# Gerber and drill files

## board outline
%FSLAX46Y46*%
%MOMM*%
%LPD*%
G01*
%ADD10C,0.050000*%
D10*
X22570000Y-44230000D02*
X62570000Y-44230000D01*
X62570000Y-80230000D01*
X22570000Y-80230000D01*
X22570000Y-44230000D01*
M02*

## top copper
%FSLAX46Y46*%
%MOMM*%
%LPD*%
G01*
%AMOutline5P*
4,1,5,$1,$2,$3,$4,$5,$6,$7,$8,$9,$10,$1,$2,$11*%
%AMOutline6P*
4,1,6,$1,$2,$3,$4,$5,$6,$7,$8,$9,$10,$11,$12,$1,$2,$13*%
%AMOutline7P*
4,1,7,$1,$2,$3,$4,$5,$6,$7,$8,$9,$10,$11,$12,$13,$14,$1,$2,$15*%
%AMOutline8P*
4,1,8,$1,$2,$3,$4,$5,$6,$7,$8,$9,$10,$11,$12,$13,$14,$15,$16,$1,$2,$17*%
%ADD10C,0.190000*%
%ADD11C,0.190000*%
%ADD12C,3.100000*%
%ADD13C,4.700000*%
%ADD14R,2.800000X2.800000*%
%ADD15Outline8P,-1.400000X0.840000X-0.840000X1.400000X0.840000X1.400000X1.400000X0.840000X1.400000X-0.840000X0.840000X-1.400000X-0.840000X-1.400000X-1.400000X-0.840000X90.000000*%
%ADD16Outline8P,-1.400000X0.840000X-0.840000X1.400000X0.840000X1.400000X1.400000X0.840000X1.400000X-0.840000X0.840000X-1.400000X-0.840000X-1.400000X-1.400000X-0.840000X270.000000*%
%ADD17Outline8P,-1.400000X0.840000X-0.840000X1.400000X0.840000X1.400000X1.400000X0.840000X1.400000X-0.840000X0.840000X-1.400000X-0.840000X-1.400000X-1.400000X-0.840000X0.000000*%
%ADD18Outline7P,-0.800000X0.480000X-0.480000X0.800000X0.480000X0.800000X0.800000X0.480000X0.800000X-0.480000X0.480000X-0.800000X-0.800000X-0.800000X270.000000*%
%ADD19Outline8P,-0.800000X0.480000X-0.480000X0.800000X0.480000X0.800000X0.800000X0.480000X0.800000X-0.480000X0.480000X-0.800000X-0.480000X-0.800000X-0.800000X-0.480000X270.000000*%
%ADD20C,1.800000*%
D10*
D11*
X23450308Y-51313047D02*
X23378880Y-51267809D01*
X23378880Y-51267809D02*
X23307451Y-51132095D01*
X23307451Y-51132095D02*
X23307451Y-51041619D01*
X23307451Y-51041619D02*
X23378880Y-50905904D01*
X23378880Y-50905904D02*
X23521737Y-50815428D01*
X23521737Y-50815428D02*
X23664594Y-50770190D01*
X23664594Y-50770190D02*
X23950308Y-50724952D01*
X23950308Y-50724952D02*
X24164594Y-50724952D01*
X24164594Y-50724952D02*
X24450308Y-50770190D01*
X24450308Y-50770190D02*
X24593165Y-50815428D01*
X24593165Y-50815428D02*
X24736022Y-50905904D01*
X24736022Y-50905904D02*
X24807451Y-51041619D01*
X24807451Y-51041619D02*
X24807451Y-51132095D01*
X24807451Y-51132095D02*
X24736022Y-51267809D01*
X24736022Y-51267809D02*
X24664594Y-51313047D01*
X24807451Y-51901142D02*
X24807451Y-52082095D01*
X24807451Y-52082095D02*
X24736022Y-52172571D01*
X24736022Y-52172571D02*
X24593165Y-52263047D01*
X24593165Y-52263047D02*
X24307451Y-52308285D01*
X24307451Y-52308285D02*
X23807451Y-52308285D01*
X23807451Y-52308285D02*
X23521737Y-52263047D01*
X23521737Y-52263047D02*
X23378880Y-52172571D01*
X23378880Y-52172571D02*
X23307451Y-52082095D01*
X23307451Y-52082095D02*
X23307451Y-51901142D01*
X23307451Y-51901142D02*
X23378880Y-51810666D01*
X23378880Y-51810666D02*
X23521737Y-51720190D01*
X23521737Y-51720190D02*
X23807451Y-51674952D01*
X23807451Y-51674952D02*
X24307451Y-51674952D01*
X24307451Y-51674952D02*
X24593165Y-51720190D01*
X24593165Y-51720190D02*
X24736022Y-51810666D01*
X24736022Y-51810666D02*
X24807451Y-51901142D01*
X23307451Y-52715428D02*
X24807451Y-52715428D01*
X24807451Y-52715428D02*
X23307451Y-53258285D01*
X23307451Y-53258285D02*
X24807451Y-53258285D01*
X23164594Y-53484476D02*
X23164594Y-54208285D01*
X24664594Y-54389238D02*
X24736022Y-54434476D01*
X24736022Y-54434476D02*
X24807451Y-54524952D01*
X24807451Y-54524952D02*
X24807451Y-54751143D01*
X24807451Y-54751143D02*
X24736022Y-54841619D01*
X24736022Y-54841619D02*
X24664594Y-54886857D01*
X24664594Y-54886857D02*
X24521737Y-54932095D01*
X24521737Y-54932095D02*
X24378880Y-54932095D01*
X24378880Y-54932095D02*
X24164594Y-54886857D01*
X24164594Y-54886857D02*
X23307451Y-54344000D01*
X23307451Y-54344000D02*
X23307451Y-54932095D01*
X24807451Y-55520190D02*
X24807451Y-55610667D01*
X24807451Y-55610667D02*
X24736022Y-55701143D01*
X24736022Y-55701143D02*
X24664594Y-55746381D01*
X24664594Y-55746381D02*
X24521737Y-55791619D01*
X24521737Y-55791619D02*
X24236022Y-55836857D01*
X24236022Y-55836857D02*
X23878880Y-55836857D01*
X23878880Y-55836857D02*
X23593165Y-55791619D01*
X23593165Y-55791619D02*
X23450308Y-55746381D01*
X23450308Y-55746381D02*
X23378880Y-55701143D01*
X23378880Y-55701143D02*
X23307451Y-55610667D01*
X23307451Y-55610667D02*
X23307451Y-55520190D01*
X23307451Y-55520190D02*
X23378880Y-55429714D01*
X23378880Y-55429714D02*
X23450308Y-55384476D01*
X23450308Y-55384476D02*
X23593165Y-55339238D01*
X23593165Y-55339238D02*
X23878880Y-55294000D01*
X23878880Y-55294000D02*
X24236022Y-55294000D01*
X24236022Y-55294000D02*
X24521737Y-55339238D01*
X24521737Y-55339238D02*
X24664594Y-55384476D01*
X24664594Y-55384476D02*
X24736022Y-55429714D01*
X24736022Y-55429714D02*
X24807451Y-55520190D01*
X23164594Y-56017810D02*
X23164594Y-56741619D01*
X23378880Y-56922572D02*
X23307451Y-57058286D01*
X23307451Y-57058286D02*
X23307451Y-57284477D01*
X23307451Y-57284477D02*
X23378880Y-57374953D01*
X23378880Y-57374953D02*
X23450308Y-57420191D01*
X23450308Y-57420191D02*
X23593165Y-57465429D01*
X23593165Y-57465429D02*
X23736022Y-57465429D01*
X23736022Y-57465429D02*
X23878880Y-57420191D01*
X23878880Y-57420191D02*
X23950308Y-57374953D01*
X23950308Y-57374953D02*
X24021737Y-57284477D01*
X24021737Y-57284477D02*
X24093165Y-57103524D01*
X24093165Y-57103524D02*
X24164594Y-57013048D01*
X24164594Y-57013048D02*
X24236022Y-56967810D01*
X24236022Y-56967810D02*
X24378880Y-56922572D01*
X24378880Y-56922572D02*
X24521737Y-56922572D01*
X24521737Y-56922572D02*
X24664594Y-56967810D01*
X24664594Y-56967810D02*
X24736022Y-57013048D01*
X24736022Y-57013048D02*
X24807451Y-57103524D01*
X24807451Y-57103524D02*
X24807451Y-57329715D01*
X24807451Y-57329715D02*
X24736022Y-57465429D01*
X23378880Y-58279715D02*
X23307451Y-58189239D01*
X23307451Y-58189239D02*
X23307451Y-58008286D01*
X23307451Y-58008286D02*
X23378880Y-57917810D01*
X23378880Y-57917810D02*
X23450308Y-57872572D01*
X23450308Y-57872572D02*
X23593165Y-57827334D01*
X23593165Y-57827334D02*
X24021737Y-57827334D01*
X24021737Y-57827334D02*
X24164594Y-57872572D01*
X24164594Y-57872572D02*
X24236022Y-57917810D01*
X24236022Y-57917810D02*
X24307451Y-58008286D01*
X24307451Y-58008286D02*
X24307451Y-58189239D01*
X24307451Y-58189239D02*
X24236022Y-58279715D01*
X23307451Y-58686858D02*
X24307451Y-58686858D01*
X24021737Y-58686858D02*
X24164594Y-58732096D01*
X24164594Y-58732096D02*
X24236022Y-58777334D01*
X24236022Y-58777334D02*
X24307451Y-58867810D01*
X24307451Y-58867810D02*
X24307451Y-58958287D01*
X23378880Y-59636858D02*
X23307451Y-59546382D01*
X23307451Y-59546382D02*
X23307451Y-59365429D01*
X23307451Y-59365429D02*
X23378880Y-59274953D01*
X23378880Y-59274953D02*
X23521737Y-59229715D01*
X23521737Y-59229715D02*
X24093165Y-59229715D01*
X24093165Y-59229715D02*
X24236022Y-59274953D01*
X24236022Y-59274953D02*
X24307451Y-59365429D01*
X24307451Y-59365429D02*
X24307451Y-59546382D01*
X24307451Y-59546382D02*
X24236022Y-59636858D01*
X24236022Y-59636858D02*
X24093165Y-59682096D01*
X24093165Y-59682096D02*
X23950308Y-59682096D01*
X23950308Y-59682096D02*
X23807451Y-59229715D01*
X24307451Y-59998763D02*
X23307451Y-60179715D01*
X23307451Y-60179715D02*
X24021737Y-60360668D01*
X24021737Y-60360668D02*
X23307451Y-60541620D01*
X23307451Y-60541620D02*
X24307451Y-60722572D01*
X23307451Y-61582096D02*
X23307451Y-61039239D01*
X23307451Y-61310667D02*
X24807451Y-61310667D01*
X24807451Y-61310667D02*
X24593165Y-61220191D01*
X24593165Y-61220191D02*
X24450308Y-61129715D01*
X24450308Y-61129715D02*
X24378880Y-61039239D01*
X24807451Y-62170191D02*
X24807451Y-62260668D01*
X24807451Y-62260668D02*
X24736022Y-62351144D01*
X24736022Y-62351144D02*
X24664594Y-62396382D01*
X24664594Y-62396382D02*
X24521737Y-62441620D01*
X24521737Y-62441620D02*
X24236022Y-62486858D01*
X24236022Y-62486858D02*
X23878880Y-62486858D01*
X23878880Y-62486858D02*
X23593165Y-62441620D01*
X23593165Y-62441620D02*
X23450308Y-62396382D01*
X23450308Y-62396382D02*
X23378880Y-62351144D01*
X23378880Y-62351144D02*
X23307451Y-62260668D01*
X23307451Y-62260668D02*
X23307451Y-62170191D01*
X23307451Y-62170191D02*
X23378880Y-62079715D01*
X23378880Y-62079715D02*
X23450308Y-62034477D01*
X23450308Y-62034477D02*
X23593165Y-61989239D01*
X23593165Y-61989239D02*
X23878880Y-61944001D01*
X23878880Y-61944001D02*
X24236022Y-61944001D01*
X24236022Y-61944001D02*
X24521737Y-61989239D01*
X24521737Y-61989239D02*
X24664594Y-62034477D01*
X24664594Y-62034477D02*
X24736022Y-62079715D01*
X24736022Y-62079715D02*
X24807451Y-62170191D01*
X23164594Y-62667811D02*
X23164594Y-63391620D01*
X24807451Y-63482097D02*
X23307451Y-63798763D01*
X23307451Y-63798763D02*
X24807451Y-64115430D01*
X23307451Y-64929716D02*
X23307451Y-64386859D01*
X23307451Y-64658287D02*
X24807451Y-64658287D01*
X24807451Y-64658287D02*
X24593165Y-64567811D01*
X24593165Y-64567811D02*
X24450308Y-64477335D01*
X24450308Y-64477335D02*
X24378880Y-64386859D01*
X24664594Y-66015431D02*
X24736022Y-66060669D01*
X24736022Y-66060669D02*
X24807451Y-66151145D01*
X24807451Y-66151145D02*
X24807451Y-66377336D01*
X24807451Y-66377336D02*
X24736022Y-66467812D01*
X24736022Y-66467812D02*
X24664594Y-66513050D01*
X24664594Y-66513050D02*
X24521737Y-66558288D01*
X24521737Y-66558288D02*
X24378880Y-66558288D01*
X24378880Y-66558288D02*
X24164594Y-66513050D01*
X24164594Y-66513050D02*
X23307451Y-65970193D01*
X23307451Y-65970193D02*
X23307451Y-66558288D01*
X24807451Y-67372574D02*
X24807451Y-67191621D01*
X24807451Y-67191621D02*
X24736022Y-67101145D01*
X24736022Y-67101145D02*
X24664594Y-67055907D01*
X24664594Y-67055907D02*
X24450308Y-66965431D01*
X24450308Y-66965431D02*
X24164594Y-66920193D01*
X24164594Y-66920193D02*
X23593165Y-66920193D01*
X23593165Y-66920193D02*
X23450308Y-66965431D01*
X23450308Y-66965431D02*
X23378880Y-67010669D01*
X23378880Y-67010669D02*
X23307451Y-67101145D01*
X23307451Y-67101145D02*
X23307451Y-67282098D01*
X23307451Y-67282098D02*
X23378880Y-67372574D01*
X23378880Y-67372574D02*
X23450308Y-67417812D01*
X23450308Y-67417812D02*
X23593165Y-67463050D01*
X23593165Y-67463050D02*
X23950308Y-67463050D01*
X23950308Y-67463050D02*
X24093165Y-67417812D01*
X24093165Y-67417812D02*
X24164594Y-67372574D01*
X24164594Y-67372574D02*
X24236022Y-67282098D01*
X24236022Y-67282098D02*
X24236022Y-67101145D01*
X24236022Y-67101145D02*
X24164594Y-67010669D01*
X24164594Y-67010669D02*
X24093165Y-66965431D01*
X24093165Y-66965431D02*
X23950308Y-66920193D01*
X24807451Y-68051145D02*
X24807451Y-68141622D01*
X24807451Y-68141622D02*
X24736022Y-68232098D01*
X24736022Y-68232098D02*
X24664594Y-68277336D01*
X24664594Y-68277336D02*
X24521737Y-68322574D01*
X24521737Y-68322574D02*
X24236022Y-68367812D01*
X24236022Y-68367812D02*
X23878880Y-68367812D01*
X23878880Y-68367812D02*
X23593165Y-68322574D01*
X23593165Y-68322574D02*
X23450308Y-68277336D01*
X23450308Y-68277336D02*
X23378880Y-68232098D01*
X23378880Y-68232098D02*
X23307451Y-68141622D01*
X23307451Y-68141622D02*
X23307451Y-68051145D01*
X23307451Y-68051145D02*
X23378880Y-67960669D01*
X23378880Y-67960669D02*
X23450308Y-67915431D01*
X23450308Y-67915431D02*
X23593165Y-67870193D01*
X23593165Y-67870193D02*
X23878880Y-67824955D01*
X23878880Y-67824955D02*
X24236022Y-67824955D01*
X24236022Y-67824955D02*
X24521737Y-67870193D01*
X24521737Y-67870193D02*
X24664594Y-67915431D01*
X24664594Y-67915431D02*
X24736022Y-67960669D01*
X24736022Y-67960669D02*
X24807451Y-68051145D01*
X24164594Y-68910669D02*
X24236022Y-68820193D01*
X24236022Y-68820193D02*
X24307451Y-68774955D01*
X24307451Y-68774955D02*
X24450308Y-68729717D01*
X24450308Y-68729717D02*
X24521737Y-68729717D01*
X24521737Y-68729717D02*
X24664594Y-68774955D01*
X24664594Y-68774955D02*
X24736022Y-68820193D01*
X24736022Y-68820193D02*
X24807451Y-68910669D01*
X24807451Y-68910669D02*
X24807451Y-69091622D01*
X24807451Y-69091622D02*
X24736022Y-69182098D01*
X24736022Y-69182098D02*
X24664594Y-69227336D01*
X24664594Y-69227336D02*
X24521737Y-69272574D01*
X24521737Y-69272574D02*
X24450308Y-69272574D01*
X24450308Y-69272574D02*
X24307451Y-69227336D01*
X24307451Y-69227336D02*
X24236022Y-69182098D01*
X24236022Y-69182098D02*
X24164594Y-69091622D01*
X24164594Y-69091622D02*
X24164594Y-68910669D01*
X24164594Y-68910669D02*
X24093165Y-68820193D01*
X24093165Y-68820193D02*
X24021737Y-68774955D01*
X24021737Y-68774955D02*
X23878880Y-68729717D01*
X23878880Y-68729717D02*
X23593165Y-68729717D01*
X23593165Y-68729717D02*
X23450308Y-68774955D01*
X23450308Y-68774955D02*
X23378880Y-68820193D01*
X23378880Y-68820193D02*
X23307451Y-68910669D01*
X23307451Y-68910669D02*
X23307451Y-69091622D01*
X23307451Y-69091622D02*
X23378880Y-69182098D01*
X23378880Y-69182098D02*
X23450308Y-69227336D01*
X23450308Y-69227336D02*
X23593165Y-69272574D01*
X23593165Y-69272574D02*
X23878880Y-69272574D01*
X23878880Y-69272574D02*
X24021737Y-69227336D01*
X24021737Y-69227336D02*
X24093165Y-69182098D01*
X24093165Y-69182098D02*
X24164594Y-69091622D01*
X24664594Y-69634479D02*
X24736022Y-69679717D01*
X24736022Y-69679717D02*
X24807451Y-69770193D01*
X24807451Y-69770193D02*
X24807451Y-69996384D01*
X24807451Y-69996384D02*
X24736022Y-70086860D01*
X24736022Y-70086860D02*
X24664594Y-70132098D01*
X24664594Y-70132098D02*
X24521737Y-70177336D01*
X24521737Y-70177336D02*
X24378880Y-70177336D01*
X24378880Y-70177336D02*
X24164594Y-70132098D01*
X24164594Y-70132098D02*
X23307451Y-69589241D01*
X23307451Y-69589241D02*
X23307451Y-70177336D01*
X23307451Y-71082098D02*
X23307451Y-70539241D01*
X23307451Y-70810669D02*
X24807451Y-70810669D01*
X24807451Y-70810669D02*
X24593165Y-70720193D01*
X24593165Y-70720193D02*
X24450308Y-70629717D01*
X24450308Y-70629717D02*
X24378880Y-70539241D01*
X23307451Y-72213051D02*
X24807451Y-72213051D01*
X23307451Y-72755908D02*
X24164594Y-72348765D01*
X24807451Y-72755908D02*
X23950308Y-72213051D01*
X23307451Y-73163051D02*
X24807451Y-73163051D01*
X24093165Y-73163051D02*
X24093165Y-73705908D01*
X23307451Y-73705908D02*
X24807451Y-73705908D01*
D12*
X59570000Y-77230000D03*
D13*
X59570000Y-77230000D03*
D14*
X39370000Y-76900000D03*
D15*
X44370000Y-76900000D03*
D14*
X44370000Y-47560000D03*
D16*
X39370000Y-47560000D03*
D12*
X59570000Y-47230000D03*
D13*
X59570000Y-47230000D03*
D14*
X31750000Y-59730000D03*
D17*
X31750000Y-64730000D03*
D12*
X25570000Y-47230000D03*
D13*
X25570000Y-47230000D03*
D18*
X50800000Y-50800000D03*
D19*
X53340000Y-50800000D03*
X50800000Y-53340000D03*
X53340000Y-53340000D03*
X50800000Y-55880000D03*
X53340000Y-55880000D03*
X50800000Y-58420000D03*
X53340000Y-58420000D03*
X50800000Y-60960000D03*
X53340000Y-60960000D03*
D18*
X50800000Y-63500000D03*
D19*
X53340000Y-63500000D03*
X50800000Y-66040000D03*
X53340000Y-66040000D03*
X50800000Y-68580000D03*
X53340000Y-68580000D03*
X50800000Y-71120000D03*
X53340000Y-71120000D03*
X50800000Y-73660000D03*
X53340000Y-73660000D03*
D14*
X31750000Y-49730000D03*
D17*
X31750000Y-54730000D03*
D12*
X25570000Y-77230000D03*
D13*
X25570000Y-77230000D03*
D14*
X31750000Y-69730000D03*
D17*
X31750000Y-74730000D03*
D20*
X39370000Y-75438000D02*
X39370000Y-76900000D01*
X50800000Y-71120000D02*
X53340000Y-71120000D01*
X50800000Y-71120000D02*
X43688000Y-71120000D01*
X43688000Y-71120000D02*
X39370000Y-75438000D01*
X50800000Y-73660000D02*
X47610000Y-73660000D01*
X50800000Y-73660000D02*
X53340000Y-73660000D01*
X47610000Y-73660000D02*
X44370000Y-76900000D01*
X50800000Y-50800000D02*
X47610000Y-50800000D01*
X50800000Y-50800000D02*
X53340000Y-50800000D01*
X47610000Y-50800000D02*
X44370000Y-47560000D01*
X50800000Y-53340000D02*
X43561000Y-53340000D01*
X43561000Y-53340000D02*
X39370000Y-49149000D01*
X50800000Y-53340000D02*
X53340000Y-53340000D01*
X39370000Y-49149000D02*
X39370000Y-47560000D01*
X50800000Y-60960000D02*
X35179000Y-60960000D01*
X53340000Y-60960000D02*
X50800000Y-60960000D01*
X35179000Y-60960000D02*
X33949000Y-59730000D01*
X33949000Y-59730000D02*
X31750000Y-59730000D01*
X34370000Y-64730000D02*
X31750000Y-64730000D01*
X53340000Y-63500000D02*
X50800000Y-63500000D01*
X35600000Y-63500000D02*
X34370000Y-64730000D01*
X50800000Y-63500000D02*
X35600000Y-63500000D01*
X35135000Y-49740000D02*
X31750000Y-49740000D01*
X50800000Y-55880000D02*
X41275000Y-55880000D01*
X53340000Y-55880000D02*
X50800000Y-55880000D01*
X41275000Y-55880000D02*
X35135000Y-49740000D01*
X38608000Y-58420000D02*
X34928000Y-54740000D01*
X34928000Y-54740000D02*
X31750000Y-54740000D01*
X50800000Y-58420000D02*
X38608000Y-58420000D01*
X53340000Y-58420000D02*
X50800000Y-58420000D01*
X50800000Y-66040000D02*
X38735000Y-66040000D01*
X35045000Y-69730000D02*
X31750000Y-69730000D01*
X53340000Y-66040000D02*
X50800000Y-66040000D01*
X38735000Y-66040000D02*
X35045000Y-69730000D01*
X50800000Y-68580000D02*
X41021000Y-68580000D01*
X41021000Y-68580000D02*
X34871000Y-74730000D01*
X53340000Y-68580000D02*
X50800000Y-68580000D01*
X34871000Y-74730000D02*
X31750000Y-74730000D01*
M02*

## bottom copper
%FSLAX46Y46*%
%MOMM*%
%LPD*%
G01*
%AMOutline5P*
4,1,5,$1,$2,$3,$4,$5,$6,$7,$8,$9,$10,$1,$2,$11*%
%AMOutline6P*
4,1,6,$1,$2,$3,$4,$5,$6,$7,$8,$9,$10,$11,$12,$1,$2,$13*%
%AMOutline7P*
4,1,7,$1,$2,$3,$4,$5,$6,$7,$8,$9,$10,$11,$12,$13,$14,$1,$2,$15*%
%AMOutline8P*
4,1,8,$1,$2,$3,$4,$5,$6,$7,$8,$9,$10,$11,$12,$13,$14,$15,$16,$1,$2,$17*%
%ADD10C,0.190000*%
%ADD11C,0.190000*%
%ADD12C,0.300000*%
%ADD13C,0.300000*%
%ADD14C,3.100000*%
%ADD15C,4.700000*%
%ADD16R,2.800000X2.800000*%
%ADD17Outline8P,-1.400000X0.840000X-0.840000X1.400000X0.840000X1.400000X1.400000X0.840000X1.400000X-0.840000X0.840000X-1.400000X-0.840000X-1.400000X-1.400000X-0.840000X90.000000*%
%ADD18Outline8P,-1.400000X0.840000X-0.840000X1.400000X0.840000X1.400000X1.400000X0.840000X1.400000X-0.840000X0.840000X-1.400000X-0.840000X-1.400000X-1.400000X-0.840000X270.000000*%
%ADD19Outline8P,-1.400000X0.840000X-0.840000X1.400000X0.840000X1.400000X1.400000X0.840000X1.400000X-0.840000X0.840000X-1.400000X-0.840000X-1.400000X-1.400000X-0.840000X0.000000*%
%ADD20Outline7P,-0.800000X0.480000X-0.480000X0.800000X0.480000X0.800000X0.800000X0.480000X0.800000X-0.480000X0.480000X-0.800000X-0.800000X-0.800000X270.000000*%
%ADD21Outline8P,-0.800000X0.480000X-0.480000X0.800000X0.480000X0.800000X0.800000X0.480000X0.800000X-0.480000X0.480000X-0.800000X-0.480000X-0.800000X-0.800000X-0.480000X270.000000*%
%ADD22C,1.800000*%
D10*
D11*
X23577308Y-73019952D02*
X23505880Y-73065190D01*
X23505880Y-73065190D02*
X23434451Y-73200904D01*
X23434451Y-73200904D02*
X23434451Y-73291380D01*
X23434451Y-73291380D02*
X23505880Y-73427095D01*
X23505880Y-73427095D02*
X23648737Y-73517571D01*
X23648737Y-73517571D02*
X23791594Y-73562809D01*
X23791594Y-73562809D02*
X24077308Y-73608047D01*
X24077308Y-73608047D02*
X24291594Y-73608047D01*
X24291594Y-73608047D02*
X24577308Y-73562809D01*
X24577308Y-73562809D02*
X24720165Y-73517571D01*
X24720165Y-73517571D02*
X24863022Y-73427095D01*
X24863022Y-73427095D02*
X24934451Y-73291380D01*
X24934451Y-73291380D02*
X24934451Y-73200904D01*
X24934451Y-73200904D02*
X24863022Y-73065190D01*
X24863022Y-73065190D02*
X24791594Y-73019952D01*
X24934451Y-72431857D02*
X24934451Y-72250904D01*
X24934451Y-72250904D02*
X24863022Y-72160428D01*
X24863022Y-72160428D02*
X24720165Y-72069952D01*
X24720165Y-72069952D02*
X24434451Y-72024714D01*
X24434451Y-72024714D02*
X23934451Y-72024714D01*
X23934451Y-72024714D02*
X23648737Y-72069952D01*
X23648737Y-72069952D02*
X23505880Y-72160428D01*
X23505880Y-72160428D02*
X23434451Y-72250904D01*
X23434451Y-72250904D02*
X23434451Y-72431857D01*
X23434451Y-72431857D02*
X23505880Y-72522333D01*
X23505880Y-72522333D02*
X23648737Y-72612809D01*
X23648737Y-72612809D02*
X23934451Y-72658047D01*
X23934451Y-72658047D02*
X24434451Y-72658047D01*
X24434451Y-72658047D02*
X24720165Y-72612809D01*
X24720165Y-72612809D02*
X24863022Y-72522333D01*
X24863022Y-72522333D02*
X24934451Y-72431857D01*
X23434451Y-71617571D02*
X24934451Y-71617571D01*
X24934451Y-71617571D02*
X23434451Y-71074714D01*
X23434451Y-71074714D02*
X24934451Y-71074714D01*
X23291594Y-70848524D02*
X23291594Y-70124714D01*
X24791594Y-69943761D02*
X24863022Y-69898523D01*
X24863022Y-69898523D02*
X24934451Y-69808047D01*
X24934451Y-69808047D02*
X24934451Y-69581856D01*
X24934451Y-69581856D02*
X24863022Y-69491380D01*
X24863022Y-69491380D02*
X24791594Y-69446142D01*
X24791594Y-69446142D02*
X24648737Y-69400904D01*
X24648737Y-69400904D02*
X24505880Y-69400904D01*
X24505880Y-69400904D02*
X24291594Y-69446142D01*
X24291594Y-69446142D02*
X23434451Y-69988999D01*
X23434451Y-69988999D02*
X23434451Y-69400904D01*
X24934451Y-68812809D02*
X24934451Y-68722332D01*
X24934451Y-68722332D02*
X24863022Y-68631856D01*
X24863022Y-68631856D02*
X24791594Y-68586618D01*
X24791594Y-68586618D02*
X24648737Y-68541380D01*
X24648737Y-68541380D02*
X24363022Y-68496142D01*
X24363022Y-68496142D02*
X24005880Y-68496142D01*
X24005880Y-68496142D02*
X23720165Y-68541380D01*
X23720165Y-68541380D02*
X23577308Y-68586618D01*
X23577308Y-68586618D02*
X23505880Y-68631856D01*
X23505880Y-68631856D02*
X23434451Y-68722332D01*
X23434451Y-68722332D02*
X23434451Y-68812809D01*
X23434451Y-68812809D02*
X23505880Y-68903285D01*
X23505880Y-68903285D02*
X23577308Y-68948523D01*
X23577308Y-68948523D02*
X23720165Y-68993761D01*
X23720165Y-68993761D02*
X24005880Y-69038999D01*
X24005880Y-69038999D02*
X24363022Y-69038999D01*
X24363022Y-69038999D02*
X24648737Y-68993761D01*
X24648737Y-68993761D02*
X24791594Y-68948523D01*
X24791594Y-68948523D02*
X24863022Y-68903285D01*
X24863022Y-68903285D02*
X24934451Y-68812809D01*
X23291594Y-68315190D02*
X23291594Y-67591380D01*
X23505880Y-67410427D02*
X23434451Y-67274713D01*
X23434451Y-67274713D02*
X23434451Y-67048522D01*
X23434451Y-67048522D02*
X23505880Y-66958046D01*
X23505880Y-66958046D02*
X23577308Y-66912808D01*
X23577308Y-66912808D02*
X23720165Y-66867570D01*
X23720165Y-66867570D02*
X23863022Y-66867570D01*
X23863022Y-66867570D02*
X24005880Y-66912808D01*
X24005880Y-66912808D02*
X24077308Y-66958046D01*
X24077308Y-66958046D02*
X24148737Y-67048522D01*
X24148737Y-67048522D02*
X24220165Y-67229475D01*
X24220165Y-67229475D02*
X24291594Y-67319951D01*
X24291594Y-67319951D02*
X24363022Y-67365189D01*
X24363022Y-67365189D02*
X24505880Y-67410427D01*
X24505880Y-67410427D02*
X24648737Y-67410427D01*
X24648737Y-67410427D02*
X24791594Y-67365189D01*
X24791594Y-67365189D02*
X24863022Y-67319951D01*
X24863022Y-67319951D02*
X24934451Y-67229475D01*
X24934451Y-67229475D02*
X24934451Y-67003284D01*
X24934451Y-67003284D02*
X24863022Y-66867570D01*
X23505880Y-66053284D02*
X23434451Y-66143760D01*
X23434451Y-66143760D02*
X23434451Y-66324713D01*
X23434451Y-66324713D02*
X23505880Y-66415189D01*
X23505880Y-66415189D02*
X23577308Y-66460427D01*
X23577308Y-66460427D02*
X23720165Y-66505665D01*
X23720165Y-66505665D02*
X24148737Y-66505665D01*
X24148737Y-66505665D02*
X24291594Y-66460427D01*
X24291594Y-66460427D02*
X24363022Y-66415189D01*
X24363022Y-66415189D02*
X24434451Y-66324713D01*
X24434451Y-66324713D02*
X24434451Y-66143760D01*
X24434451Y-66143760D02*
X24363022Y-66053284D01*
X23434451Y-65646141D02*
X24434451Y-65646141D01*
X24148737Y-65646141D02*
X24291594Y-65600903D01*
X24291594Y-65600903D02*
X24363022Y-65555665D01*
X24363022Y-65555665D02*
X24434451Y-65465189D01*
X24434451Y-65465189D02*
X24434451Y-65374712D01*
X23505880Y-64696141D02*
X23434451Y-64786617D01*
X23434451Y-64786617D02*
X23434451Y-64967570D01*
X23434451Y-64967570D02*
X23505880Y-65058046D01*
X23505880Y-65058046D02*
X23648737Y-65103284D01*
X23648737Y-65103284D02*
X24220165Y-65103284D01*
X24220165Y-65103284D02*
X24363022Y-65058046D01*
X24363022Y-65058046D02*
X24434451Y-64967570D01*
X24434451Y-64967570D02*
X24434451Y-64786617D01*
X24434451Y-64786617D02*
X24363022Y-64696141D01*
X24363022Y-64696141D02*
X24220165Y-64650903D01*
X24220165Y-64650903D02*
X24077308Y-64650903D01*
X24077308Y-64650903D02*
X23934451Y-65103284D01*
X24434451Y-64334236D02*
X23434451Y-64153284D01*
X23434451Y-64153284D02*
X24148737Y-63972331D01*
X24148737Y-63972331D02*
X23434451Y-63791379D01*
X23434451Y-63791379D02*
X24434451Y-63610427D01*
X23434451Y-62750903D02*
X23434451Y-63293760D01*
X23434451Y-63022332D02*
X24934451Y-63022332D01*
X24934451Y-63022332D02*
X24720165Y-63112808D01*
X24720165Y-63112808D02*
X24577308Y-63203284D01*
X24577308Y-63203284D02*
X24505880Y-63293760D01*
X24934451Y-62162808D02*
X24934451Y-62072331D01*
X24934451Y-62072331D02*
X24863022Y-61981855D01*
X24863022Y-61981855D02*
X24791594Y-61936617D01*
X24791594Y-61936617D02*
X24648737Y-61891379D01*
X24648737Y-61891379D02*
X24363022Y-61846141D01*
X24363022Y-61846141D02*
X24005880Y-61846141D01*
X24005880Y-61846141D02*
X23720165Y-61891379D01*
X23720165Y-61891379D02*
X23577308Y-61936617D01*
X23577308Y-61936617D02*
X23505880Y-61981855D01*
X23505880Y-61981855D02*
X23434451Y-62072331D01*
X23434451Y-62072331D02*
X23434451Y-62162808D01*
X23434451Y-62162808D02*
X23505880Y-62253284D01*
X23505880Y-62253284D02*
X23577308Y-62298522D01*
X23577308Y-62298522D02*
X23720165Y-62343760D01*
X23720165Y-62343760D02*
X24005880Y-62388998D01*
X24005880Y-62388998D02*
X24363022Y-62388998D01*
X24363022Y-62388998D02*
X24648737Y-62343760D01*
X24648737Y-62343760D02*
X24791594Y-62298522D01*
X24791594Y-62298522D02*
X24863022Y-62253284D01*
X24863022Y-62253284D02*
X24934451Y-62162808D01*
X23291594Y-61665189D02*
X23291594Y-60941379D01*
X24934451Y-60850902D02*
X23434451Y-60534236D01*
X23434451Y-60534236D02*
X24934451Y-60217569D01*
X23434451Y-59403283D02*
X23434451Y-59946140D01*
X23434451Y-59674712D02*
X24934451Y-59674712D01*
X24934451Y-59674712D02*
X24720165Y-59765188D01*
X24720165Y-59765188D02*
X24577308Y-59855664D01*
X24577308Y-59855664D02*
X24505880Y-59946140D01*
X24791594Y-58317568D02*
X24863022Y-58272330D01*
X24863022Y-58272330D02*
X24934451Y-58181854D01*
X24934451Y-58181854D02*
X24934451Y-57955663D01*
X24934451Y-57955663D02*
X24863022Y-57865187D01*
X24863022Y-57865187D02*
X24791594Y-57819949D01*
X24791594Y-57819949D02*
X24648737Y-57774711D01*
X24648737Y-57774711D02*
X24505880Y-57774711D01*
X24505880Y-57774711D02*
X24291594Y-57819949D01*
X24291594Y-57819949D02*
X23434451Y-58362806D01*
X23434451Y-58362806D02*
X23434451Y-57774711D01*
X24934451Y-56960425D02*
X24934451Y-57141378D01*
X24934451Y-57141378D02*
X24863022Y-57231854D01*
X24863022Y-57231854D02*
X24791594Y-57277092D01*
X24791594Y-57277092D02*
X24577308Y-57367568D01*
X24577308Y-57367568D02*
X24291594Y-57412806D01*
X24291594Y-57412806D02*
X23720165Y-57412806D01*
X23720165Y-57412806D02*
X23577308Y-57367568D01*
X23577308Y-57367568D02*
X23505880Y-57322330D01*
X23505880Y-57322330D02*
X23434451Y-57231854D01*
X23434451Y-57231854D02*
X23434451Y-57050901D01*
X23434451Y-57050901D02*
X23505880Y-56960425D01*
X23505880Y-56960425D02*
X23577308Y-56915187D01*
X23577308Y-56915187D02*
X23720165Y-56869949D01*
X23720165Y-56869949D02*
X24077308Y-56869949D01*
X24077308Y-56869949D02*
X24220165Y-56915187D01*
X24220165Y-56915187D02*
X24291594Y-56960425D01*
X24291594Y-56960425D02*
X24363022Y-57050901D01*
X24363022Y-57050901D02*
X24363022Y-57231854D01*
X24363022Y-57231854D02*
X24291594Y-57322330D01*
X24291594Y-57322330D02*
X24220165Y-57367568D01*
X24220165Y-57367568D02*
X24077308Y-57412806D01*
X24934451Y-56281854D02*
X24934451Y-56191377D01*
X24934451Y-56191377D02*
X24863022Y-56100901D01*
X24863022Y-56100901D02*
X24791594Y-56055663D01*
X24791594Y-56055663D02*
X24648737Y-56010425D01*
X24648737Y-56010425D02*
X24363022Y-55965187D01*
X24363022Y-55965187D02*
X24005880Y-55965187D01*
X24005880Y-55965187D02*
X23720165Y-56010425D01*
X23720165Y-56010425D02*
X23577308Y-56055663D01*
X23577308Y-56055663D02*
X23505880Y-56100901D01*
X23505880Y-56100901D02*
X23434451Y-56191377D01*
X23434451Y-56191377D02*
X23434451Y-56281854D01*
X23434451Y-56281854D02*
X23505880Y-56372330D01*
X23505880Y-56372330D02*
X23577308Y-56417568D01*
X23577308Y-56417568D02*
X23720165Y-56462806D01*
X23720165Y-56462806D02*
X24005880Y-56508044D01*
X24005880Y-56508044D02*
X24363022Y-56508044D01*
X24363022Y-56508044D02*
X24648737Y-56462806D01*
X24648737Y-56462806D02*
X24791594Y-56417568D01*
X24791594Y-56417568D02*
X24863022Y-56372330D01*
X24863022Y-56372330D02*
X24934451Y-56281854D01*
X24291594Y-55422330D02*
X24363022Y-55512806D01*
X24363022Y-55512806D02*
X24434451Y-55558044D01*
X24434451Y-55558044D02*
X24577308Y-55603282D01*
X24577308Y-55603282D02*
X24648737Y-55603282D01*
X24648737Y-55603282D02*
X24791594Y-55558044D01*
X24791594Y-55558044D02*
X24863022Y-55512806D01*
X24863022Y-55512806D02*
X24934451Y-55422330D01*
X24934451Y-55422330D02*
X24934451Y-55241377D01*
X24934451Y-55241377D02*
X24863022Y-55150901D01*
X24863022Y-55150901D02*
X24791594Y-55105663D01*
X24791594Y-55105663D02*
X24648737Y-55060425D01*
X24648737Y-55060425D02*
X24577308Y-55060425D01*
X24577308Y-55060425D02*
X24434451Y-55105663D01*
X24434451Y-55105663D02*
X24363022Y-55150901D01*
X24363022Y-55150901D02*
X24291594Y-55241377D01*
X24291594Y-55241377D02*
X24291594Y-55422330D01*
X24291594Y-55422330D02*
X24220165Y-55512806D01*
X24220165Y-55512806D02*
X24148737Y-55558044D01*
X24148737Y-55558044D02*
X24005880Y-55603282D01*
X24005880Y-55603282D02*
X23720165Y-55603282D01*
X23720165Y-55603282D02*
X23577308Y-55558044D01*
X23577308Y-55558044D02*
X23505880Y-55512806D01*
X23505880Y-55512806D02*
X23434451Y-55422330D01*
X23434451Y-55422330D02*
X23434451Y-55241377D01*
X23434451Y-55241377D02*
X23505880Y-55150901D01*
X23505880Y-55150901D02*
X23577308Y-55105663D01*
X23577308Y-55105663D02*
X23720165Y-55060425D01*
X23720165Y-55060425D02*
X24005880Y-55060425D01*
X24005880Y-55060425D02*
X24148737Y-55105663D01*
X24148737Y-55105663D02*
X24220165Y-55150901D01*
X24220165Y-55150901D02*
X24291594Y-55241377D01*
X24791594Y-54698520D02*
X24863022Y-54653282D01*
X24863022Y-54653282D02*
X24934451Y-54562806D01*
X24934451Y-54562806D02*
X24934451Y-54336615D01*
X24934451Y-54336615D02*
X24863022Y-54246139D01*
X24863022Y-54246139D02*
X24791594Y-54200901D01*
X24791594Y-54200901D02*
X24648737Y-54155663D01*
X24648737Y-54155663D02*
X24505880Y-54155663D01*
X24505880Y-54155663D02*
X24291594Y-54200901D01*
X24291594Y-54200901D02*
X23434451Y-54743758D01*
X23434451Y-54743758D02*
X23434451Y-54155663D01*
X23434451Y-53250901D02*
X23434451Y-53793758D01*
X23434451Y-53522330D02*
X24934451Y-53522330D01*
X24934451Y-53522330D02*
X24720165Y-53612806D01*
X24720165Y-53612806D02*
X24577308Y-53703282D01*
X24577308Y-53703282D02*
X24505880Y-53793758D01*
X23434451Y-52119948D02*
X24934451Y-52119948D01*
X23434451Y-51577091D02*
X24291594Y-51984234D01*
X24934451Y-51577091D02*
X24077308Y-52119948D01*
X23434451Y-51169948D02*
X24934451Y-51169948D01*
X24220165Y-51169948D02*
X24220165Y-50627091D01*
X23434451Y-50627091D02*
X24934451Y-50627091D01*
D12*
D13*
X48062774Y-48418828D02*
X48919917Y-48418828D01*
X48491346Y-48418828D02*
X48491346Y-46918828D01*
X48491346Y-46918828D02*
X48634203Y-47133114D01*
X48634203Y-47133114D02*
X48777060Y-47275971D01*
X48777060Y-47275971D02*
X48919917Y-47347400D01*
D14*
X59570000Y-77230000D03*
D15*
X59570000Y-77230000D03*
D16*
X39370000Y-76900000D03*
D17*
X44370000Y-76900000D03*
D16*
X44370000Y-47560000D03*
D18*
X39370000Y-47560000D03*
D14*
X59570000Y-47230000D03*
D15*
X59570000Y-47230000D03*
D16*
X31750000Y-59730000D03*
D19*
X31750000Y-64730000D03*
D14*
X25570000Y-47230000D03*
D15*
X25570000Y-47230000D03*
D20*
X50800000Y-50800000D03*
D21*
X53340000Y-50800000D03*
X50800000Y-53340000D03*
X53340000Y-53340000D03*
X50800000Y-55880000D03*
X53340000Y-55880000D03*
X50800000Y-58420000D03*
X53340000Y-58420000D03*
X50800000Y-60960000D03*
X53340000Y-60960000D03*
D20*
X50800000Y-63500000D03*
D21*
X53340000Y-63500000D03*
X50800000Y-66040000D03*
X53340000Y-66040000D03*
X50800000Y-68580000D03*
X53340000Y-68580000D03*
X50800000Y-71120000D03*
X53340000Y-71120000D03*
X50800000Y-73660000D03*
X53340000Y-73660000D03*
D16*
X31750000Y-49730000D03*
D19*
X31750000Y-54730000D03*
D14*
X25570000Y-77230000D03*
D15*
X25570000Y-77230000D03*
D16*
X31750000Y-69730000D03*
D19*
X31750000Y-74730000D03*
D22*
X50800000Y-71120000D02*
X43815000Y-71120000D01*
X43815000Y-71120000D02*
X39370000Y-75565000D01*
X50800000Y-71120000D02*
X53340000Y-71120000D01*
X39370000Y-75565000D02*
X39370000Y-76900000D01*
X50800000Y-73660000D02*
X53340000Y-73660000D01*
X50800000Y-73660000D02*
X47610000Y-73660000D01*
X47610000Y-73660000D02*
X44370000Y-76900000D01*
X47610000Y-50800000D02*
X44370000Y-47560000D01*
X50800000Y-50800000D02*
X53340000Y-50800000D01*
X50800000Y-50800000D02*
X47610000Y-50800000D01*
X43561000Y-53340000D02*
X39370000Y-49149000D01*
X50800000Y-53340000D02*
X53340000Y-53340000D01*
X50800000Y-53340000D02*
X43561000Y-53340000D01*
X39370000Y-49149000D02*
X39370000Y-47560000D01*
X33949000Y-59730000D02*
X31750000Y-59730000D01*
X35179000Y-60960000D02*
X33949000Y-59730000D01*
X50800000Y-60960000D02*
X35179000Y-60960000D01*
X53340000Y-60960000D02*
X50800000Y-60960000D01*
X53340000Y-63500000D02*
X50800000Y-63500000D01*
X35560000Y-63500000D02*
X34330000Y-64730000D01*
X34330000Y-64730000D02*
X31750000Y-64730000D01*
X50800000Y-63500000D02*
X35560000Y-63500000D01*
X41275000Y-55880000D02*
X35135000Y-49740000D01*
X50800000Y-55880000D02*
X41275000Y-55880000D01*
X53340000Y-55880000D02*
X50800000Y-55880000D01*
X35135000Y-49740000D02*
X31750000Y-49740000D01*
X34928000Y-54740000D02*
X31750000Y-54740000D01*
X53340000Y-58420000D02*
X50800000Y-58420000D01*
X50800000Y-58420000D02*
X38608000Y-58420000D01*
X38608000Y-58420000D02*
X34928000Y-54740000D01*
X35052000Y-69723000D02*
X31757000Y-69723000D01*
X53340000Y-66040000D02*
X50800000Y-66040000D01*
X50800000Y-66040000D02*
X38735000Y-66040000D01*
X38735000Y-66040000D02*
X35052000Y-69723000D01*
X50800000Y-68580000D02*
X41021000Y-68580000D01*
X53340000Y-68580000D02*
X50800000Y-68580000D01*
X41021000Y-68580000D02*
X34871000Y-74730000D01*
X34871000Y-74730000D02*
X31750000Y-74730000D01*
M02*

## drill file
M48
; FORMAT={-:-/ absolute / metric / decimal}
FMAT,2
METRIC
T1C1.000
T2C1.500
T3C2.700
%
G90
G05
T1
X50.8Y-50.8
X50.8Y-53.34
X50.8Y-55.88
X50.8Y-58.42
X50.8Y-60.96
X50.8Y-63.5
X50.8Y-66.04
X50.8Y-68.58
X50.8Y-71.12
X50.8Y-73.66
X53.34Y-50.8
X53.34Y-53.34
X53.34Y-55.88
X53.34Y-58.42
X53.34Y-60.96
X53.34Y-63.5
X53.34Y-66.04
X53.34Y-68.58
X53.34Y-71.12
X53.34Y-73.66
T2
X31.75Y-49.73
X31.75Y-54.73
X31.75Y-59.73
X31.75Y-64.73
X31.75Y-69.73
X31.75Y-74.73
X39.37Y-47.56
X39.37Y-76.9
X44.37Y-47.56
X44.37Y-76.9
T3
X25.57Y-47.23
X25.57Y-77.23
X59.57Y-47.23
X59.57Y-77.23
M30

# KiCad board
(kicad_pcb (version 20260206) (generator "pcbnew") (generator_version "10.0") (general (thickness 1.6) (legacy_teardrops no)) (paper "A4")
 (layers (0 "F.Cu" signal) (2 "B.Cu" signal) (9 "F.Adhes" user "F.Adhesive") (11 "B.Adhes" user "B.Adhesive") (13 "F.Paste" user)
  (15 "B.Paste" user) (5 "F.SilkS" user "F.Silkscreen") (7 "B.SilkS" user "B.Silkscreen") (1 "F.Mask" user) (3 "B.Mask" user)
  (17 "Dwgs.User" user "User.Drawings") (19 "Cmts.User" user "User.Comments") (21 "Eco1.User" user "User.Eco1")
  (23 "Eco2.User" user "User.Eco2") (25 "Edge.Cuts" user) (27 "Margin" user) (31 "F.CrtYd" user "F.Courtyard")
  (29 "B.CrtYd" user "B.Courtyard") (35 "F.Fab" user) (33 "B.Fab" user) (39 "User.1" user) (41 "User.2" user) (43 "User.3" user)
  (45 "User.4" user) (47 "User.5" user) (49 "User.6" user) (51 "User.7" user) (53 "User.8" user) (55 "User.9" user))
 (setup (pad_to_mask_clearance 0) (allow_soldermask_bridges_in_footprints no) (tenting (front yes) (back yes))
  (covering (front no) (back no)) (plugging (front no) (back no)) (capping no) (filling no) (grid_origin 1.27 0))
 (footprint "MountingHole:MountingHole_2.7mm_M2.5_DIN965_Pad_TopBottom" (layer "F.Cu") (at 59.57 77.23)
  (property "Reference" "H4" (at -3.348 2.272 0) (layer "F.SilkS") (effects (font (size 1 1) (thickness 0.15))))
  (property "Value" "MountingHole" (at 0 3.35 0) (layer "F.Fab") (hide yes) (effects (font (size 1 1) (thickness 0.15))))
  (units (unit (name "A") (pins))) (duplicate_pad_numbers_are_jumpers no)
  (pad "1" thru_hole circle (at 0 0) (size 3.1 3.1) (drill 2.7) (layers "*.Cu" "*.Mask") (remove_unused_layers no))
  (pad "1" connect circle (at 0 0) (size 4.7 4.7) (layers "F.Cu" "F.Mask"))
  (pad "1" connect circle (at 0 0) (size 4.7 4.7) (layers "B.Cu" "B.Mask")))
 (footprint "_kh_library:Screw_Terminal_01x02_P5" (layer "F.Cu") (at 39.37 76.9 90)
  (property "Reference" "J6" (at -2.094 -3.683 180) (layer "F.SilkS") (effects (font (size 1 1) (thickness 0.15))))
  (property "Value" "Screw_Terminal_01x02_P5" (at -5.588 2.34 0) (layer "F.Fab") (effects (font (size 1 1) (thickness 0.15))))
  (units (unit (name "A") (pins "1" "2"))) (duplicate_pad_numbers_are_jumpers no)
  (pad "1" thru_hole rect (at 0 0 90) (size 2.8 2.8) (drill 1.5) (layers "*.Cu" "*.Mask") (remove_unused_layers no) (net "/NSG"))
  (pad "2" thru_hole roundrect (at 0 5 90) (size 2.8 2.8) (drill 1.5) (layers "*.Cu" "*.Mask") (remove_unused_layers no)
   (roundrect_rratio 0) (chamfer_ratio 0.2) (chamfer top_left top_right bottom_left bottom_right) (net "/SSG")))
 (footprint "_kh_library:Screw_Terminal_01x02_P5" (layer "F.Cu") (at 44.37 47.56 -90)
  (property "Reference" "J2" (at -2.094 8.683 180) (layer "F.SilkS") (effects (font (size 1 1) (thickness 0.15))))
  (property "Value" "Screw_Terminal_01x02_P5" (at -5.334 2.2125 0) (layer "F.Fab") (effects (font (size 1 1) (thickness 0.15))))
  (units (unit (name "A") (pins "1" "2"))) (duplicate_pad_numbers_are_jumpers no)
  (pad "1" thru_hole rect (at 0 0 270) (size 2.8 2.8) (drill 1.5) (layers "*.Cu" "*.Mask") (remove_unused_layers no) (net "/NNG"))
  (pad "2" thru_hole roundrect (at 0 5 270) (size 2.8 2.8) (drill 1.5) (layers "*.Cu" "*.Mask") (remove_unused_layers no)
   (roundrect_rratio 0) (chamfer_ratio 0.2) (chamfer top_left top_right bottom_left bottom_right) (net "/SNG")))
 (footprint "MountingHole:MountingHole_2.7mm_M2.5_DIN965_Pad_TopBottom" (layer "F.Cu") (at 59.57 47.23)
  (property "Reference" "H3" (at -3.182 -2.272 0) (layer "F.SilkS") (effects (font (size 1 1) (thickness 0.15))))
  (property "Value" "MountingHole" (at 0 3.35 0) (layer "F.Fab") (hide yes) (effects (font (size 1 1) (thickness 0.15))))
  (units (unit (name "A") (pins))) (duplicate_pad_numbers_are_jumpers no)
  (pad "1" thru_hole circle (at 0 0) (size 3.1 3.1) (drill 2.7) (layers "*.Cu" "*.Mask") (remove_unused_layers no))
  (pad "1" connect circle (at 0 0) (size 4.7 4.7) (layers "F.Cu" "F.Mask"))
  (pad "1" connect circle (at 0 0) (size 4.7 4.7) (layers "B.Cu" "B.Mask")))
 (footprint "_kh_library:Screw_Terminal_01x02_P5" (layer "F.Cu") (at 31.75 59.73)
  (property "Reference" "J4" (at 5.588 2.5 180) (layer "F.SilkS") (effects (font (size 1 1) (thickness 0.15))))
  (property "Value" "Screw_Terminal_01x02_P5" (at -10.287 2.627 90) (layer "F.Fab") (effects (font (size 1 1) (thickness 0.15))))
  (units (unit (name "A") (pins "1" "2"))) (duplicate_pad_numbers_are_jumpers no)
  (pad "1" thru_hole rect (at 0 0) (size 2.8 2.8) (drill 1.5) (layers "*.Cu" "*.Mask") (remove_unused_layers no) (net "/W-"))
  (pad "2" thru_hole roundrect (at 0 5) (size 2.8 2.8) (drill 1.5) (layers "*.Cu" "*.Mask") (remove_unused_layers no) (roundrect_rratio 0)
   (chamfer_ratio 0.2) (chamfer top_left top_right bottom_left bottom_right) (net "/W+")))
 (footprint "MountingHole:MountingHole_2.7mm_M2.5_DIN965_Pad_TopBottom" (layer "F.Cu") (at 25.57 47.23)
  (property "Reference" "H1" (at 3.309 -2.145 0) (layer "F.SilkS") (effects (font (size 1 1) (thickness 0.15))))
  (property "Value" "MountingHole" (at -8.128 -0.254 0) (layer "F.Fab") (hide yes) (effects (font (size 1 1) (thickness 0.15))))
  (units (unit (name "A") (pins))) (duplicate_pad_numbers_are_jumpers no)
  (pad "1" thru_hole circle (at 0 0) (size 3.1 3.1) (drill 2.7) (layers "*.Cu" "*.Mask") (remove_unused_layers no))
  (pad "1" connect circle (at 0 0) (size 4.7 4.7) (layers "F.Cu" "F.Mask"))
  (pad "1" connect circle (at 0 0) (size 4.7 4.7) (layers "B.Cu" "B.Mask")))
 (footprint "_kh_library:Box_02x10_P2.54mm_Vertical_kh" (layer "F.Cu") (at 50.8 50.8 -90)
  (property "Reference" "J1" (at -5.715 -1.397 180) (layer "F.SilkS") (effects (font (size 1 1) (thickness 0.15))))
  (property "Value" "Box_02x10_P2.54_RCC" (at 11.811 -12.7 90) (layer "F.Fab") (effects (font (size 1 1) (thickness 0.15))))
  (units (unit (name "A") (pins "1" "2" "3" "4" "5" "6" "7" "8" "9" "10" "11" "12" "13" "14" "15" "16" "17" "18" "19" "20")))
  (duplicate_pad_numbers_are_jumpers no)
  (pad "1" thru_hole roundrect (at 0 0 270) (size 1.6 1.6) (drill 1) (layers "*.Cu" "*.Mask") (remove_unused_layers no) (roundrect_rratio 0)
   (chamfer_ratio 0.2) (chamfer top_left top_right bottom_right) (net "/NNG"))
  (pad "2" thru_hole roundrect (at 0 -2.54 270) (size 1.6 1.6) (drill 1) (layers "*.Cu" "*.Mask") (remove_unused_layers no)
   (roundrect_rratio 0) (chamfer_ratio 0.2) (chamfer top_left top_right bottom_left bottom_right) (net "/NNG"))
  (pad "3" thru_hole roundrect (at 2.54 0 270) (size 1.6 1.6) (drill 1) (layers "*.Cu" "*.Mask") (remove_unused_layers no)
   (roundrect_rratio 0) (chamfer_ratio 0.2) (chamfer top_left top_right bottom_left bottom_right) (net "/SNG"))
  (pad "4" thru_hole roundrect (at 2.54 -2.54 270) (size 1.6 1.6) (drill 1) (layers "*.Cu" "*.Mask") (remove_unused_layers no)
   (roundrect_rratio 0) (chamfer_ratio 0.2) (chamfer top_left top_right bottom_left bottom_right) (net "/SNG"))
  (pad "5" thru_hole roundrect (at 5.08 0 270) (size 1.6 1.6) (drill 1) (layers "*.Cu" "*.Mask") (remove_unused_layers no)
   (roundrect_rratio 0) (chamfer_ratio 0.2) (chamfer top_left top_right bottom_left bottom_right) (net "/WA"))
  (pad "6" thru_hole roundrect (at 5.08 -2.54 270) (size 1.6 1.6) (drill 1) (layers "*.Cu" "*.Mask") (remove_unused_layers no)
   (roundrect_rratio 0) (chamfer_ratio 0.2) (chamfer top_left top_right bottom_left bottom_right) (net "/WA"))
  (pad "7" thru_hole roundrect (at 7.62 0 270) (size 1.6 1.6) (drill 1) (layers "*.Cu" "*.Mask") (remove_unused_layers no)
   (roundrect_rratio 0) (chamfer_ratio 0.2) (chamfer top_left top_right bottom_left bottom_right) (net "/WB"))
  (pad "8" thru_hole roundrect (at 7.62 -2.54 270) (size 1.6 1.6) (drill 1) (layers "*.Cu" "*.Mask") (remove_unused_layers no)
   (roundrect_rratio 0) (chamfer_ratio 0.2) (chamfer top_left top_right bottom_left bottom_right) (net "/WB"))
  (pad "9" thru_hole roundrect (at 10.16 0 270) (size 1.6 1.6) (drill 1) (layers "*.Cu" "*.Mask") (remove_unused_layers no)
   (roundrect_rratio 0) (chamfer_ratio 0.2) (chamfer top_left top_right bottom_left bottom_right) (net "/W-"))
  (pad "10" thru_hole roundrect (at 10.16 -2.54 270) (size 1.6 1.6) (drill 1) (layers "*.Cu" "*.Mask") (remove_unused_layers no)
   (roundrect_rratio 0) (chamfer_ratio 0.2) (chamfer top_left top_right bottom_left bottom_right) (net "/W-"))
  (pad "11" thru_hole roundrect (at 12.7 0 270) (size 1.6 1.6) (drill 1) (layers "*.Cu" "*.Mask") (remove_unused_layers no)
   (roundrect_rratio 0) (chamfer_ratio 0.2) (chamfer top_left top_right bottom_right) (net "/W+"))
  (pad "12" thru_hole roundrect (at 12.7 -2.54 270) (size 1.6 1.6) (drill 1) (layers "*.Cu" "*.Mask") (remove_unused_layers no)
   (roundrect_rratio 0) (chamfer_ratio 0.2) (chamfer top_left top_right bottom_left bottom_right) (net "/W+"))
  (pad "13" thru_hole roundrect (at 15.24 0 270) (size 1.6 1.6) (drill 1) (layers "*.Cu" "*.Mask") (remove_unused_layers no)
   (roundrect_rratio 0) (chamfer_ratio 0.2) (chamfer top_left top_right bottom_left bottom_right) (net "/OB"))
  (pad "14" thru_hole roundrect (at 15.24 -2.54 270) (size 1.6 1.6) (drill 1) (layers "*.Cu" "*.Mask") (remove_unused_layers no)
   (roundrect_rratio 0) (chamfer_ratio 0.2) (chamfer top_left top_right bottom_left bottom_right) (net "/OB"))
  (pad "15" thru_hole roundrect (at 17.78 0 270) (size 1.6 1.6) (drill 1) (layers "*.Cu" "*.Mask") (remove_unused_layers no)
   (roundrect_rratio 0) (chamfer_ratio 0.2) (chamfer top_left top_right bottom_left bottom_right) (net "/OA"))
  (pad "16" thru_hole roundrect (at 17.78 -2.54 270) (size 1.6 1.6) (drill 1) (layers "*.Cu" "*.Mask") (remove_unused_layers no)
   (roundrect_rratio 0) (chamfer_ratio 0.2) (chamfer top_left top_right bottom_left bottom_right) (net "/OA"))
  (pad "17" thru_hole roundrect (at 20.32 0 270) (size 1.6 1.6) (drill 1) (layers "*.Cu" "*.Mask") (remove_unused_layers no)
   (roundrect_rratio 0) (chamfer_ratio 0.2) (chamfer top_left top_right bottom_left bottom_right) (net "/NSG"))
  (pad "18" thru_hole roundrect (at 20.32 -2.54 270) (size 1.6 1.6) (drill 1) (layers "*.Cu" "*.Mask") (remove_unused_layers no)
   (roundrect_rratio 0) (chamfer_ratio 0.2) (chamfer top_left top_right bottom_left bottom_right) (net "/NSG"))
  (pad "19" thru_hole roundrect (at 22.86 0 270) (size 1.6 1.6) (drill 1) (layers "*.Cu" "*.Mask") (remove_unused_layers no)
   (roundrect_rratio 0) (chamfer_ratio 0.2) (chamfer top_left top_right bottom_left bottom_right) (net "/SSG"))
  (pad "20" thru_hole roundrect (at 22.86 -2.54 270) (size 1.6 1.6) (drill 1) (layers "*.Cu" "*.Mask") (remove_unused_layers no)
   (roundrect_rratio 0) (chamfer_ratio 0.2) (chamfer top_left top_right bottom_left bottom_right) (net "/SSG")))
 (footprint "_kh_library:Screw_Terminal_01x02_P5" (layer "F.Cu") (at 31.75 49.73)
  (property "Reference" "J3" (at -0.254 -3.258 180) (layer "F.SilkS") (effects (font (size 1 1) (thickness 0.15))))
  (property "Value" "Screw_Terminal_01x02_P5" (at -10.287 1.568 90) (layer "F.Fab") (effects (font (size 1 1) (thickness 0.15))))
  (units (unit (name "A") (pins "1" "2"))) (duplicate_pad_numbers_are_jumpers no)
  (pad "1" thru_hole rect (at 0 0) (size 2.8 2.8) (drill 1.5) (layers "*.Cu" "*.Mask") (remove_unused_layers no) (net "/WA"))
  (pad "2" thru_hole roundrect (at 0 5) (size 2.8 2.8) (drill 1.5) (layers "*.Cu" "*.Mask") (remove_unused_layers no) (roundrect_rratio 0)
   (chamfer_ratio 0.2) (chamfer top_left top_right bottom_left bottom_right) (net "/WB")))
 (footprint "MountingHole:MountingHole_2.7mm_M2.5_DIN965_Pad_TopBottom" (layer "F.Cu") (at 25.57 77.23)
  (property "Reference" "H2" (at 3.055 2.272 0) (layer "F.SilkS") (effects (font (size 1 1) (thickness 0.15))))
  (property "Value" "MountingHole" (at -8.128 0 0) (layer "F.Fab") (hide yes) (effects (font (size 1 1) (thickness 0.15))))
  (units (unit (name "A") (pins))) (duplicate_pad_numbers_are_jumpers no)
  (pad "1" thru_hole circle (at 0 0) (size 3.1 3.1) (drill 2.7) (layers "*.Cu" "*.Mask") (remove_unused_layers no))
  (pad "1" connect circle (at 0 0) (size 4.7 4.7) (layers "F.Cu" "F.Mask"))
  (pad "1" connect circle (at 0 0) (size 4.7 4.7) (layers "B.Cu" "B.Mask")))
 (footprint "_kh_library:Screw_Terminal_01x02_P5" (layer "F.Cu") (at 31.75 69.73)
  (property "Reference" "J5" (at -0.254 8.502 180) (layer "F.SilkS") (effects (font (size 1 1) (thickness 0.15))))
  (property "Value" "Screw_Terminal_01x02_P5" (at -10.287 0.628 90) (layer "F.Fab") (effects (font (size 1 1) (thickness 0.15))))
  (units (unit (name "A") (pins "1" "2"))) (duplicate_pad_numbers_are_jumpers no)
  (pad "1" thru_hole rect (at 0 0) (size 2.8 2.8) (drill 1.5) (layers "*.Cu" "*.Mask") (remove_unused_layers no) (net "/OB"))
  (pad "2" thru_hole roundrect (at 0 5) (size 2.8 2.8) (drill 1.5) (layers "*.Cu" "*.Mask") (remove_unused_layers no) (roundrect_rratio 0)
   (chamfer_ratio 0.2) (chamfer top_left top_right bottom_left bottom_right) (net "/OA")))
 (gr_rect (start 22.57 44.23) (end 62.57 80.23) (stroke (width 0.05) (type default)) (fill no) (layer "Edge.Cuts"))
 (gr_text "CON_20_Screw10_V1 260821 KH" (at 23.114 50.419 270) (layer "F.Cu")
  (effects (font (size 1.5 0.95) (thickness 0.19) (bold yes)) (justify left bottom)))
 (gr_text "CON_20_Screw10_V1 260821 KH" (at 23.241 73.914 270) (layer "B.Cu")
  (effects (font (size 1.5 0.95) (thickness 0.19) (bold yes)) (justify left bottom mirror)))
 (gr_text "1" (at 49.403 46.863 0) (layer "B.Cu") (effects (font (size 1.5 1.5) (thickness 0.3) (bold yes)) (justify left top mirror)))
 (segment (start 39.37 75.438) (end 39.37 76.9) (width 1.8) (layer "F.Cu") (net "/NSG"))
 (segment (start 50.8 71.12) (end 53.34 71.12) (width 1.8) (layer "F.Cu") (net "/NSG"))
 (segment (start 50.8 71.12) (end 43.688 71.12) (width 1.8) (layer "F.Cu") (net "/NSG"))
 (segment (start 43.688 71.12) (end 39.37 75.438) (width 1.8) (layer "F.Cu") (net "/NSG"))
 (segment (start 50.8 71.12) (end 43.815 71.12) (width 1.8) (layer "B.Cu") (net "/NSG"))
 (segment (start 43.815 71.12) (end 39.37 75.565) (width 1.8) (layer "B.Cu") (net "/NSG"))
 (segment (start 50.8 71.12) (end 53.34 71.12) (width 1.8) (layer "B.Cu") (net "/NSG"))
 (segment (start 39.37 75.565) (end 39.37 76.9) (width 1.8) (layer "B.Cu") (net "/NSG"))
 (segment (start 50.8 73.66) (end 47.61 73.66) (width 1.8) (layer "F.Cu") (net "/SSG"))
 (segment (start 50.8 73.66) (end 53.34 73.66) (width 1.8) (layer "F.Cu") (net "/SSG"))
 (segment (start 47.61 73.66) (end 44.37 76.9) (width 1.8) (layer "F.Cu") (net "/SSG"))
 (segment (start 50.8 73.66) (end 53.34 73.66) (width 1.8) (layer "B.Cu") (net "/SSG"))
 (segment (start 50.8 73.66) (end 47.61 73.66) (width 1.8) (layer "B.Cu") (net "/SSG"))
 (segment (start 47.61 73.66) (end 44.37 76.9) (width 1.8) (layer "B.Cu") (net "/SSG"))
 (segment (start 50.8 50.8) (end 47.61 50.8) (width 1.8) (layer "F.Cu") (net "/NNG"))
 (segment (start 50.8 50.8) (end 53.34 50.8) (width 1.8) (layer "F.Cu") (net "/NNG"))
 (segment (start 47.61 50.8) (end 44.37 47.56) (width 1.8) (layer "F.Cu") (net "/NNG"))
 (segment (start 47.61 50.8) (end 44.37 47.56) (width 1.8) (layer "B.Cu") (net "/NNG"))
 (segment (start 50.8 50.8) (end 53.34 50.8) (width 1.8) (layer "B.Cu") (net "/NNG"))
 (segment (start 50.8 50.8) (end 47.61 50.8) (width 1.8) (layer "B.Cu") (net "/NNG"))
 (segment (start 50.8 53.34) (end 43.561 53.34) (width 1.8) (layer "F.Cu") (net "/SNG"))
 (segment (start 43.561 53.34) (end 39.37 49.149) (width 1.8) (layer "F.Cu") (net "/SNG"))
 (segment (start 50.8 53.34) (end 53.34 53.34) (width 1.8) (layer "F.Cu") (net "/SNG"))
 (segment (start 39.37 49.149) (end 39.37 47.56) (width 1.8) (layer "F.Cu") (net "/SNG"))
 (segment (start 43.561 53.34) (end 39.37 49.149) (width 1.8) (layer "B.Cu") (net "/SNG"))
 (segment (start 50.8 53.34) (end 53.34 53.34) (width 1.8) (layer "B.Cu") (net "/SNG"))
 (segment (start 50.8 53.34) (end 43.561 53.34) (width 1.8) (layer "B.Cu") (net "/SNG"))
 (segment (start 39.37 49.149) (end 39.37 47.56) (width 1.8) (layer "B.Cu") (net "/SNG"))
 (segment (start 50.8 60.96) (end 35.179 60.96) (width 1.8) (layer "F.Cu") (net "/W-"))
 (segment (start 53.34 60.96) (end 50.8 60.96) (width 1.8) (layer "F.Cu") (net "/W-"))
 (segment (start 35.179 60.96) (end 33.949 59.73) (width 1.8) (layer "F.Cu") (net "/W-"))
 (segment (start 33.949 59.73) (end 31.75 59.73) (width 1.8) (layer "F.Cu") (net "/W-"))
 (segment (start 33.949 59.73) (end 31.75 59.73) (width 1.8) (layer "B.Cu") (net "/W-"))
 (segment (start 35.179 60.96) (end 33.949 59.73) (width 1.8) (layer "B.Cu") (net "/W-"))
 (segment (start 50.8 60.96) (end 35.179 60.96) (width 1.8) (layer "B.Cu") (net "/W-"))
 (segment (start 53.34 60.96) (end 50.8 60.96) (width 1.8) (layer "B.Cu") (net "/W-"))
 (segment (start 34.37 64.73) (end 31.75 64.73) (width 1.8) (layer "F.Cu") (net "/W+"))
 (segment (start 53.34 63.5) (end 50.8 63.5) (width 1.8) (layer "F.Cu") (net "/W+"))
 (segment (start 35.6 63.5) (end 34.37 64.73) (width 1.8) (layer "F.Cu") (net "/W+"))
 (segment (start 50.8 63.5) (end 35.6 63.5) (width 1.8) (layer "F.Cu") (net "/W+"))
 (segment (start 53.34 63.5) (end 50.8 63.5) (width 1.8) (layer "B.Cu") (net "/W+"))
 (segment (start 35.56 63.5) (end 34.33 64.73) (width 1.8) (layer "B.Cu") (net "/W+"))
 (segment (start 34.33 64.73) (end 31.75 64.73) (width 1.8) (layer "B.Cu") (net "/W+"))
 (segment (start 50.8 63.5) (end 35.56 63.5) (width 1.8) (layer "B.Cu") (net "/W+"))
 (segment (start 35.135 49.74) (end 31.75 49.74) (width 1.8) (layer "F.Cu") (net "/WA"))
 (segment (start 50.8 55.88) (end 41.275 55.88) (width 1.8) (layer "F.Cu") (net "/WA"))
 (segment (start 53.34 55.88) (end 50.8 55.88) (width 1.8) (layer "F.Cu") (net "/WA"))
 (segment (start 41.275 55.88) (end 35.135 49.74) (width 1.8) (layer "F.Cu") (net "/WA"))
 (segment (start 41.275 55.88) (end 35.135 49.74) (width 1.8) (layer "B.Cu") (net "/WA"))
 (segment (start 50.8 55.88) (end 41.275 55.88) (width 1.8) (layer "B.Cu") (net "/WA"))
 (segment (start 53.34 55.88) (end 50.8 55.88) (width 1.8) (layer "B.Cu") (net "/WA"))
 (segment (start 35.135 49.74) (end 31.75 49.74) (width 1.8) (layer "B.Cu") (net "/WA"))
 (segment (start 38.608 58.42) (end 34.928 54.74) (width 1.8) (layer "F.Cu") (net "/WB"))
 (segment (start 34.928 54.74) (end 31.75 54.74) (width 1.8) (layer "F.Cu") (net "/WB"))
 (segment (start 50.8 58.42) (end 38.608 58.42) (width 1.8) (layer "F.Cu") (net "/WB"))
 (segment (start 53.34 58.42) (end 50.8 58.42) (width 1.8) (layer "F.Cu") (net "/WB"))
 (segment (start 34.928 54.74) (end 31.75 54.74) (width 1.8) (layer "B.Cu") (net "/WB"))
 (segment (start 53.34 58.42) (end 50.8 58.42) (width 1.8) (layer "B.Cu") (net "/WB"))
 (segment (start 50.8 58.42) (end 38.608 58.42) (width 1.8) (layer "B.Cu") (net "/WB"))
 (segment (start 38.608 58.42) (end 34.928 54.74) (width 1.8) (layer "B.Cu") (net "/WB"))
 (segment (start 50.8 66.04) (end 38.735 66.04) (width 1.8) (layer "F.Cu") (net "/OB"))
 (segment (start 35.045 69.73) (end 31.75 69.73) (width 1.8) (layer "F.Cu") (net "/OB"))
 (segment (start 53.34 66.04) (end 50.8 66.04) (width 1.8) (layer "F.Cu") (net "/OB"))
 (segment (start 38.735 66.04) (end 35.045 69.73) (width 1.8) (layer "F.Cu") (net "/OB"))
 (segment (start 35.052 69.723) (end 31.757 69.723) (width 1.8) (layer "B.Cu") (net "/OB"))
 (segment (start 53.34 66.04) (end 50.8 66.04) (width 1.8) (layer "B.Cu") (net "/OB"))
 (segment (start 50.8 66.04) (end 38.735 66.04) (width 1.8) (layer "B.Cu") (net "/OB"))
 (segment (start 38.735 66.04) (end 35.052 69.723) (width 1.8) (layer "B.Cu") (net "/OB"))
 (segment (start 50.8 68.58) (end 41.021 68.58) (width 1.8) (layer "F.Cu") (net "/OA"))
 (segment (start 41.021 68.58) (end 34.871 74.73) (width 1.8) (layer "F.Cu") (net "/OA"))
 (segment (start 53.34 68.58) (end 50.8 68.58) (width 1.8) (layer "F.Cu") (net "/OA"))
 (segment (start 34.871 74.73) (end 31.75 74.73) (width 1.8) (layer "F.Cu") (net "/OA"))
 (segment (start 50.8 68.58) (end 41.021 68.58) (width 1.8) (layer "B.Cu") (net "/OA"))
 (segment (start 53.34 68.58) (end 50.8 68.58) (width 1.8) (layer "B.Cu") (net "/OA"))
 (segment (start 41.021 68.58) (end 34.871 74.73) (width 1.8) (layer "B.Cu") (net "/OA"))
 (segment (start 34.871 74.73) (end 31.75 74.73) (width 1.8) (layer "B.Cu") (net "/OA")))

